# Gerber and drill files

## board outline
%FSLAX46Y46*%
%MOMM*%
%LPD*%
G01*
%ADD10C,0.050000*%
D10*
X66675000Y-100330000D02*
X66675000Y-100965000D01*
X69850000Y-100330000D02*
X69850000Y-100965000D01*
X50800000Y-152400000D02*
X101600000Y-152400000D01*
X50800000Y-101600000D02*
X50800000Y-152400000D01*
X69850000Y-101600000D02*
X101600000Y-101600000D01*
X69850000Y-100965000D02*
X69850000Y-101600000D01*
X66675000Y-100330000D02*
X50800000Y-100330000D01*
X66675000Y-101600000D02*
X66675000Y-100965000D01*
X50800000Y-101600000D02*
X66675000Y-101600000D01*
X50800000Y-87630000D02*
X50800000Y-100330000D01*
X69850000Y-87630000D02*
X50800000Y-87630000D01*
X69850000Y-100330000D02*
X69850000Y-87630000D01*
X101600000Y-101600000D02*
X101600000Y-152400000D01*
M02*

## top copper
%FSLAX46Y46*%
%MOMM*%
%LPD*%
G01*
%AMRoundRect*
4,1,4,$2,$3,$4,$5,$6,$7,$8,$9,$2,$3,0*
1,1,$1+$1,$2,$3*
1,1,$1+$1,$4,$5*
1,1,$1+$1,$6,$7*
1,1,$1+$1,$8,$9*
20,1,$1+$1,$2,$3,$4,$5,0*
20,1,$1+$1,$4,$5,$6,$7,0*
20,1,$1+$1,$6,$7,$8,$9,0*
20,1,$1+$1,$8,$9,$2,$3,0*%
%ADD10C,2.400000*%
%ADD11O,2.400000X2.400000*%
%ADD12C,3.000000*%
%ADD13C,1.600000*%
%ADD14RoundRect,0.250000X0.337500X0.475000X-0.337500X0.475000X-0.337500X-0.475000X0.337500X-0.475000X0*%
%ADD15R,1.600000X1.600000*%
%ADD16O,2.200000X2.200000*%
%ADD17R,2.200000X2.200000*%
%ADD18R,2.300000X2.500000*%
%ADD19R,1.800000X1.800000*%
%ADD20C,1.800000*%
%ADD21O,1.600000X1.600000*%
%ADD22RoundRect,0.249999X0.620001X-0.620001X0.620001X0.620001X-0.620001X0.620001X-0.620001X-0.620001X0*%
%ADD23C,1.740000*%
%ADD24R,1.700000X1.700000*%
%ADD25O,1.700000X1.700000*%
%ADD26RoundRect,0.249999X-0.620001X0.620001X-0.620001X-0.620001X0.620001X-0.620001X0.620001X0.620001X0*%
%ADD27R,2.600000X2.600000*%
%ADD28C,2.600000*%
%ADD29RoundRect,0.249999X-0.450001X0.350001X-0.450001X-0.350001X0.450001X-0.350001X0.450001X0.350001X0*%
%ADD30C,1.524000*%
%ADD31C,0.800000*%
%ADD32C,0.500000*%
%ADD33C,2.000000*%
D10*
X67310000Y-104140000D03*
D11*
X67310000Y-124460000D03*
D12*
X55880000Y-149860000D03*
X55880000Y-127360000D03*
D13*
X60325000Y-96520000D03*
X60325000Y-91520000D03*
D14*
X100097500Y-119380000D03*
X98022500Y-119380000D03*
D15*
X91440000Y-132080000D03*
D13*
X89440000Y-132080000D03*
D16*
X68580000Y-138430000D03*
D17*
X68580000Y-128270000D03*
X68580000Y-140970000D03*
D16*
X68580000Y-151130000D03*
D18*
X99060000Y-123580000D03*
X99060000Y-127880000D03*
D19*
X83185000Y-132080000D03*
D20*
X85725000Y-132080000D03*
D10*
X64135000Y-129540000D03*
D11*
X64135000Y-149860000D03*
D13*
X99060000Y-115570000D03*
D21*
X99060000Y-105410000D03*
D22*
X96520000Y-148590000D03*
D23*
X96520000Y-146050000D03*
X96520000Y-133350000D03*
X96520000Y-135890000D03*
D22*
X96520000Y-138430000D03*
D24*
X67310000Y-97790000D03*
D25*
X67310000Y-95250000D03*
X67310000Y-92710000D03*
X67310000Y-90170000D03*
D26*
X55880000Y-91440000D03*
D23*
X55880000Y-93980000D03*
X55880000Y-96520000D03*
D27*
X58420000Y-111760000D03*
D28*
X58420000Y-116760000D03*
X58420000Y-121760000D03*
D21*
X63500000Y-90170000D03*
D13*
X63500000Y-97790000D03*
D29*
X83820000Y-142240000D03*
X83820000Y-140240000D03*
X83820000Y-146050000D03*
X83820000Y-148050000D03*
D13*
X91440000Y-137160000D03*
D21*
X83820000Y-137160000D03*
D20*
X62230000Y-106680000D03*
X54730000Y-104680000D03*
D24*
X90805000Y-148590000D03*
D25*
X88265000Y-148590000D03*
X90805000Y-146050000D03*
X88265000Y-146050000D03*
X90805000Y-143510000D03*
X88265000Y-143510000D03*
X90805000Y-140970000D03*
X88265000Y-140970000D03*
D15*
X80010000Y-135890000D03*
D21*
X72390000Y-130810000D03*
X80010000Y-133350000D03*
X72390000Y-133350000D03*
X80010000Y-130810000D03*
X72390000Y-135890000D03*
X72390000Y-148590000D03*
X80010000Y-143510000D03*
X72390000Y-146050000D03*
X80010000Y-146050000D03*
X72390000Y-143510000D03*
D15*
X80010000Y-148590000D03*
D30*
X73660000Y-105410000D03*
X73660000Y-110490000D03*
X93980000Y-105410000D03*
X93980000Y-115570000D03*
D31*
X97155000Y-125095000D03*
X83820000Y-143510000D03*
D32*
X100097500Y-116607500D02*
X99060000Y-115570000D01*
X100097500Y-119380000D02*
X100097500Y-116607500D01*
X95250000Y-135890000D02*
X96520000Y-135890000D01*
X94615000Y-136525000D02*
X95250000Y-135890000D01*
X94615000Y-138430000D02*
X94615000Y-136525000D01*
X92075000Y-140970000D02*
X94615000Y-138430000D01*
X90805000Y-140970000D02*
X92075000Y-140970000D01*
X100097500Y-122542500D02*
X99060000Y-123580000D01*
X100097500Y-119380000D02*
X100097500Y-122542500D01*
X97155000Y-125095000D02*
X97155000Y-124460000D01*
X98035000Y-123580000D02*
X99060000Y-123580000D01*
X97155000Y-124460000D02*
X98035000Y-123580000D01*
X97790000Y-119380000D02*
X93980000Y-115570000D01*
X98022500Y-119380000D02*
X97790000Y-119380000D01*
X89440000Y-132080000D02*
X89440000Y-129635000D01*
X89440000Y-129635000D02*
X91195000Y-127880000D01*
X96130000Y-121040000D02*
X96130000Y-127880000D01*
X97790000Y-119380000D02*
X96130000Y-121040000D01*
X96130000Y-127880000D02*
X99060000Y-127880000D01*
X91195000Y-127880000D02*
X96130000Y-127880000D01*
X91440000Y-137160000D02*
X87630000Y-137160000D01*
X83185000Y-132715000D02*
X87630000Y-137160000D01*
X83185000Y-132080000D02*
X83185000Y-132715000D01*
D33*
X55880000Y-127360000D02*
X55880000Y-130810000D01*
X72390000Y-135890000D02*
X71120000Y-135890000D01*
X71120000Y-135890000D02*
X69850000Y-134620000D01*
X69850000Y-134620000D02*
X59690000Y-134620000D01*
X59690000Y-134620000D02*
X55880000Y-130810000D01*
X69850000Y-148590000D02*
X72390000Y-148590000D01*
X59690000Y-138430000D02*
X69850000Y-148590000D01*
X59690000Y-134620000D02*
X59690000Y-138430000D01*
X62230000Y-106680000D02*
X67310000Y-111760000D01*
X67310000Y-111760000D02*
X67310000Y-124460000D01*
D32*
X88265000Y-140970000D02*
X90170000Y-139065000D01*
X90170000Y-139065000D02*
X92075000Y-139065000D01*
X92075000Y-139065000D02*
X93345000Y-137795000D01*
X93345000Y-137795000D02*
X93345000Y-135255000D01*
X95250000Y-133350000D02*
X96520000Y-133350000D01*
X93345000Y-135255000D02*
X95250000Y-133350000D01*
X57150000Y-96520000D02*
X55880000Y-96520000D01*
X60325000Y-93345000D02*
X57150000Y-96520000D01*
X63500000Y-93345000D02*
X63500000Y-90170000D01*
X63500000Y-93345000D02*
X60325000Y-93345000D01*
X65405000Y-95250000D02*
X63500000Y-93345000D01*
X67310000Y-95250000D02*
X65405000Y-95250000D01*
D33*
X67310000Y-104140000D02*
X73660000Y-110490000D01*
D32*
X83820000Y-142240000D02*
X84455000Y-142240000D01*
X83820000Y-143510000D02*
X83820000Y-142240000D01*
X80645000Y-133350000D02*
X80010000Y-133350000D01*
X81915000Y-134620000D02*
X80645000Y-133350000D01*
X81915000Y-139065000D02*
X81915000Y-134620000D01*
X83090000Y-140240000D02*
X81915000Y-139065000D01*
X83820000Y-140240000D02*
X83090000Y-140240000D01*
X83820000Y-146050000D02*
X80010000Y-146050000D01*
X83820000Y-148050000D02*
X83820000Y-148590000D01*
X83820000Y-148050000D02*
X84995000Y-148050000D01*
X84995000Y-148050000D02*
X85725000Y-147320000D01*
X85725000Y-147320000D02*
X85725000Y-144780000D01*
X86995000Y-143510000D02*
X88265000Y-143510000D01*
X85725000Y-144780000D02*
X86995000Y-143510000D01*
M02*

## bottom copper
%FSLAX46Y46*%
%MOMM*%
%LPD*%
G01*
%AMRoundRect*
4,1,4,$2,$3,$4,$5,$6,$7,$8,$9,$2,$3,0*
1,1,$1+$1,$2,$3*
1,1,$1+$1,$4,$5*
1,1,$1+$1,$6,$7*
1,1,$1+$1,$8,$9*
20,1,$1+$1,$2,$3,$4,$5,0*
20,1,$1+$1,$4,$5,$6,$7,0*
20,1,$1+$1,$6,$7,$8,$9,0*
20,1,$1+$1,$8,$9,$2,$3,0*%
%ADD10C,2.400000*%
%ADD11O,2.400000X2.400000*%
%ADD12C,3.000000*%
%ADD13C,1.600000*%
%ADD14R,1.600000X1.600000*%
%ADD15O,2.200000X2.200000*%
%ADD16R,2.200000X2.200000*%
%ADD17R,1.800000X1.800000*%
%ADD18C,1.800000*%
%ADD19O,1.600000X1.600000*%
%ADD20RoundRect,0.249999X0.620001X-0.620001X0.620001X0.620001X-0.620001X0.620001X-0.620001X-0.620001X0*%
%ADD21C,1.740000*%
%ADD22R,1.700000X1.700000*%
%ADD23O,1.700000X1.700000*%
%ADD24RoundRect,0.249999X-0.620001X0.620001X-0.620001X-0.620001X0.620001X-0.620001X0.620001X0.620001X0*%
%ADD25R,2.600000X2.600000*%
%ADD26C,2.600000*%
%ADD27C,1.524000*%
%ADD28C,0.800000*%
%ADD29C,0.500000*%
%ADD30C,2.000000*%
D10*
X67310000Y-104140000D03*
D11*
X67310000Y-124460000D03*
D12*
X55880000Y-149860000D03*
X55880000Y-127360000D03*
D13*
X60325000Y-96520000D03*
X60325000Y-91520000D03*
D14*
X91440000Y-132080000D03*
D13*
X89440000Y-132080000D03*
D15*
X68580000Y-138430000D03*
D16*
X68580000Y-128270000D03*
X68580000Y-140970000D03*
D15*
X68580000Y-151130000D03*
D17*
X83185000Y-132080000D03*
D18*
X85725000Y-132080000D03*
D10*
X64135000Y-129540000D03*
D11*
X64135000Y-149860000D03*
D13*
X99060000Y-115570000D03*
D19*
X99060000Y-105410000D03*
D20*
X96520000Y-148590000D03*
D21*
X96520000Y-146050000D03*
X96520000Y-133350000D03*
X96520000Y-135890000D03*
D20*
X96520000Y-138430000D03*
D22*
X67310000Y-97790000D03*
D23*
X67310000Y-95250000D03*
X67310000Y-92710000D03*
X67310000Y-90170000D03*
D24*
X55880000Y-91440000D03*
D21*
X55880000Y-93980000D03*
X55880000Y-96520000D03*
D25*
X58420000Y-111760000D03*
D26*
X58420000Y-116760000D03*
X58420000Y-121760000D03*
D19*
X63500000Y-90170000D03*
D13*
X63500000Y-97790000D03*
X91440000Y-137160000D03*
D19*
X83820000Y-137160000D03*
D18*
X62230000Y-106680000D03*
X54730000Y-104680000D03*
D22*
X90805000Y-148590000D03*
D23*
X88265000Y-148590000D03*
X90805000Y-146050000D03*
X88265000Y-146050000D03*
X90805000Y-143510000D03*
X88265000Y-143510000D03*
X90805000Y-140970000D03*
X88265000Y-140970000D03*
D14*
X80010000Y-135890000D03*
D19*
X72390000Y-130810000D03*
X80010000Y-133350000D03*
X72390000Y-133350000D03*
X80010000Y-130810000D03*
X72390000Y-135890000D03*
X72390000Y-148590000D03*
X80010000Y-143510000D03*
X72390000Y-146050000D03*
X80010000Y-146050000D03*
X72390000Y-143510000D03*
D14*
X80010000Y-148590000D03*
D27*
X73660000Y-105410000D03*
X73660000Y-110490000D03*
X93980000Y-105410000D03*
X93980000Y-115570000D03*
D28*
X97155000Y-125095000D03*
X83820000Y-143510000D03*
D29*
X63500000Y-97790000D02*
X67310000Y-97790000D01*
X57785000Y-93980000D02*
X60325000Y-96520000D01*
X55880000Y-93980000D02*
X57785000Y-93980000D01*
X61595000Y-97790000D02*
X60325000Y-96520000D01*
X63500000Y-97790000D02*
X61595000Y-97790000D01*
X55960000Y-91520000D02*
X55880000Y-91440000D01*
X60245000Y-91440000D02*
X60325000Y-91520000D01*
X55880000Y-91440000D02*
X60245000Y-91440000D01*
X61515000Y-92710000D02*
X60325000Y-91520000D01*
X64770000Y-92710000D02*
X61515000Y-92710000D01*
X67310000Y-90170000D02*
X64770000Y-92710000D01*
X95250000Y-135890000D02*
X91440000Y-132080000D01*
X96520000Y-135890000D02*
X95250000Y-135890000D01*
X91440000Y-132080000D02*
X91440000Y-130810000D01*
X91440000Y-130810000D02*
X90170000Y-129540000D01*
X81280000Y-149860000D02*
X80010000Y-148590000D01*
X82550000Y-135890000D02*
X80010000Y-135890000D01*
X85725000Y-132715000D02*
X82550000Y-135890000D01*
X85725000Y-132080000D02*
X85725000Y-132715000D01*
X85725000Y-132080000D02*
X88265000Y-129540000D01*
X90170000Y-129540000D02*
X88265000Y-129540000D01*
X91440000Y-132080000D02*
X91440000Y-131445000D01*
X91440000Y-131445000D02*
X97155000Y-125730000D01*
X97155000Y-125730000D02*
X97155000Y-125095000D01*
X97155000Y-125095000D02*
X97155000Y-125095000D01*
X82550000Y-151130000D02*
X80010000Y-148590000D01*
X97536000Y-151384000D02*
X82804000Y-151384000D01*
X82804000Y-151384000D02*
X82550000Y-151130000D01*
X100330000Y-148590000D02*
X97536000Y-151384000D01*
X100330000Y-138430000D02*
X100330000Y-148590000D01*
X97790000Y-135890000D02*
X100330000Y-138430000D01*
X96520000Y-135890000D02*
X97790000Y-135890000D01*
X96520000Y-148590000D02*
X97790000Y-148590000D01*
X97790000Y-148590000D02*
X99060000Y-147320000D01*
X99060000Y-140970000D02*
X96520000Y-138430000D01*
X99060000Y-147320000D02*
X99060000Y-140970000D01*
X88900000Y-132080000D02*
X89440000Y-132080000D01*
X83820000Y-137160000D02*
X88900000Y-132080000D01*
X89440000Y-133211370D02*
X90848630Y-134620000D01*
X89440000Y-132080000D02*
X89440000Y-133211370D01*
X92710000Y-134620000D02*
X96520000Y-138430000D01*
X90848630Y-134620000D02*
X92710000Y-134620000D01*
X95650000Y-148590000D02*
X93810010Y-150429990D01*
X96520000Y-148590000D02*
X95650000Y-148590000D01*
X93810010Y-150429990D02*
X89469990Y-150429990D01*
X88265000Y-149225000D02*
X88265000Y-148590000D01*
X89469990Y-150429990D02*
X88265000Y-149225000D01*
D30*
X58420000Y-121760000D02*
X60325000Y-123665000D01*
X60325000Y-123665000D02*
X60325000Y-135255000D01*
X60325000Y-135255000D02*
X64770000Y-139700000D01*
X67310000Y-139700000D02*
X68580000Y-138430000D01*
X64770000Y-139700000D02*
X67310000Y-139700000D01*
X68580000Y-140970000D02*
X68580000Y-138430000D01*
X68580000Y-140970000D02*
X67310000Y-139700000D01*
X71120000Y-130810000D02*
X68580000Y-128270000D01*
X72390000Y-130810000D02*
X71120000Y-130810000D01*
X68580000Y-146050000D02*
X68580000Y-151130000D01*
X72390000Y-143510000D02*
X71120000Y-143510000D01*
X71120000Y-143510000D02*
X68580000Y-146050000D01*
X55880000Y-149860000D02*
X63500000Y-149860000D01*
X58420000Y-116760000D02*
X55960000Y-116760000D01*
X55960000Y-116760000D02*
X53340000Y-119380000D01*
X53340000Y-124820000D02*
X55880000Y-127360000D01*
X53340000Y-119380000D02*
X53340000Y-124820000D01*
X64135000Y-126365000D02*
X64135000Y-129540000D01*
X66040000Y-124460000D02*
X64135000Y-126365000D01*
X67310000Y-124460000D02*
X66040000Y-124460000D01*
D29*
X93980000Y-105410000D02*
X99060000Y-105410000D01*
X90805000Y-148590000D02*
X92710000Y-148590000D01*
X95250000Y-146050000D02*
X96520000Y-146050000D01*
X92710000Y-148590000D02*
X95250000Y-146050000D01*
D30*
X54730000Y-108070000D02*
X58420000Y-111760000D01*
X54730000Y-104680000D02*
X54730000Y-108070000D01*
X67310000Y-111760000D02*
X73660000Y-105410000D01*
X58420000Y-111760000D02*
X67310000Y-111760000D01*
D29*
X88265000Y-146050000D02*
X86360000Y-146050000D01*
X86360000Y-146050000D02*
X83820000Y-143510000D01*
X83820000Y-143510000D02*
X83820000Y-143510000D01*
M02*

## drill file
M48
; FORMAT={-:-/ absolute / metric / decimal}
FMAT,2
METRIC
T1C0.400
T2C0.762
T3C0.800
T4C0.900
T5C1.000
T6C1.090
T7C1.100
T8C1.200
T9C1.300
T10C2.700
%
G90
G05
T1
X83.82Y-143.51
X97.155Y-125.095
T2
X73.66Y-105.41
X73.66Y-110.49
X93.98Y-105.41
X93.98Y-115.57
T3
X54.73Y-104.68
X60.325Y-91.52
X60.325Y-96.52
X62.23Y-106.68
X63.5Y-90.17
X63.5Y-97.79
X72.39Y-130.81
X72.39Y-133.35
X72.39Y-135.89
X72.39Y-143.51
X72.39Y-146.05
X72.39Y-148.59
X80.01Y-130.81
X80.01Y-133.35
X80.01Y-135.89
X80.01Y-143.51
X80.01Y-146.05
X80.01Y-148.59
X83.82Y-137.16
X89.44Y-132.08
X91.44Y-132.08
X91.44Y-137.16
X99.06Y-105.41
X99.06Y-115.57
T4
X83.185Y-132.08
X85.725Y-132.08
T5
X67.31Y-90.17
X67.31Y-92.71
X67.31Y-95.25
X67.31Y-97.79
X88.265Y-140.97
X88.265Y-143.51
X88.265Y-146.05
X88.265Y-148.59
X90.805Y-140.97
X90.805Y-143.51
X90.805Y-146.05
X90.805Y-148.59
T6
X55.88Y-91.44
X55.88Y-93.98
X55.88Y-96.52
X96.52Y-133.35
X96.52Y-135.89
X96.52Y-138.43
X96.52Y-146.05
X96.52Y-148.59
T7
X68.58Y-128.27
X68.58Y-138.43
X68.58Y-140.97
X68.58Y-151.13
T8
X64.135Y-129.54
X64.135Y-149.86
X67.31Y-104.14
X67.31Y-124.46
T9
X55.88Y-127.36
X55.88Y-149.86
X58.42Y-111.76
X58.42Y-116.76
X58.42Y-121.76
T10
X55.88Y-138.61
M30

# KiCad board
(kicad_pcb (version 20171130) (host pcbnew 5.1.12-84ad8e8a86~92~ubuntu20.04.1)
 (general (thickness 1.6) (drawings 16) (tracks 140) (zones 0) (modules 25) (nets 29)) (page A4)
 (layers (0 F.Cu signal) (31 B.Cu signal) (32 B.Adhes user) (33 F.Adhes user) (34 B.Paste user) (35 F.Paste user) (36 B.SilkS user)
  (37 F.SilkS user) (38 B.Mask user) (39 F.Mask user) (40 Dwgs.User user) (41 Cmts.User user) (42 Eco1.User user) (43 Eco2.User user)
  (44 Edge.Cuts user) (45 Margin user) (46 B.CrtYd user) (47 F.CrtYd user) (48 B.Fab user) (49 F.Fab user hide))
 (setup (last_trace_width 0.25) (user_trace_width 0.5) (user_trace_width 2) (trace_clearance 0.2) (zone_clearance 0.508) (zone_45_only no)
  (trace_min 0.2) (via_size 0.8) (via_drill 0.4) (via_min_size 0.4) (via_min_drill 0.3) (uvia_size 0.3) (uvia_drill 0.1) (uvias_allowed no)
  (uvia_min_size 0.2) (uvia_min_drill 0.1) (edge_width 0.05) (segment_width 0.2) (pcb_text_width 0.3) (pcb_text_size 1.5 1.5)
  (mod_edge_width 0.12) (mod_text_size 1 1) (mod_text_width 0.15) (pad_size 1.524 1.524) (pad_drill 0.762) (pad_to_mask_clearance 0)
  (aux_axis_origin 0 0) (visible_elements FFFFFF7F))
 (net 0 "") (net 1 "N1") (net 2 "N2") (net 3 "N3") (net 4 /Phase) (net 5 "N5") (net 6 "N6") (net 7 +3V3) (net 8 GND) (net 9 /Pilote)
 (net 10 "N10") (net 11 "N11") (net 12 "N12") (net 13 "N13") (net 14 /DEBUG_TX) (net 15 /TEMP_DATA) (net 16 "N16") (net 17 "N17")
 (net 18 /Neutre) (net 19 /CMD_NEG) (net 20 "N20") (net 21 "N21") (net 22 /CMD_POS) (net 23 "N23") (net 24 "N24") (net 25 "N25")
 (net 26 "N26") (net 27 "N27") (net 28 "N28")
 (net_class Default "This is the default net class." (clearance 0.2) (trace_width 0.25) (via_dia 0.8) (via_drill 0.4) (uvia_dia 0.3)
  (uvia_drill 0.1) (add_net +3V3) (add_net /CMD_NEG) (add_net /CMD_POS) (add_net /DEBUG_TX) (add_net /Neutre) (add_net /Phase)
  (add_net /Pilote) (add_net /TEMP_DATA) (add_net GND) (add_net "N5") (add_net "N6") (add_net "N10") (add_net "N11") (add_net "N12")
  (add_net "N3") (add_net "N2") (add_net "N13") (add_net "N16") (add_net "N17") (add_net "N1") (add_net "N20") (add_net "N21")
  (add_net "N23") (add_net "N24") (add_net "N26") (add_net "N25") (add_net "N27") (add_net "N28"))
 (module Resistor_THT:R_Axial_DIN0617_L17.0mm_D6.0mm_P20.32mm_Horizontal (layer F.Cu) (at 67.31 104.14 270)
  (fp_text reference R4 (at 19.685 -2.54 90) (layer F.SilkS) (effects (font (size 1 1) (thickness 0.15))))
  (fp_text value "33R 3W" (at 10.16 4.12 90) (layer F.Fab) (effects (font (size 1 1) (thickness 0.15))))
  (pad 1 thru_hole circle (at 0 0 270) (size 2.4 2.4) (drill 1.2) (layers *.Cu *.Mask) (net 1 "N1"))
  (pad 2 thru_hole oval (at 20.32 0 270) (size 2.4 2.4) (drill 1.2) (layers *.Cu *.Mask) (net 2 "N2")))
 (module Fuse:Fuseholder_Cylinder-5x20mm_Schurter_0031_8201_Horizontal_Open (layer F.Cu) (at 55.88 149.86 90)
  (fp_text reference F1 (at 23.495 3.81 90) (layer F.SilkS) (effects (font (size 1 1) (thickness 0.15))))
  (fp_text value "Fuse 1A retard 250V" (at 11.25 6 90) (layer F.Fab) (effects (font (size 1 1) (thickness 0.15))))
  (pad 1 thru_hole circle (at 0 0 90) (size 3 3) (drill 1.3) (layers *.Cu *.Mask) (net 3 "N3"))
  (pad 2 thru_hole circle (at 22.5 0 90) (size 3 3) (drill 1.3) (layers *.Cu *.Mask) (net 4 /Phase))
  (pad "" np_thru_hole circle (at 11.25 0 90) (size 2.7 2.7) (drill 2.7) (layers *.Cu *.Mask)))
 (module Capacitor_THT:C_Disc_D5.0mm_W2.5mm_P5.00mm (layer F.Cu) (at 60.325 96.52 90)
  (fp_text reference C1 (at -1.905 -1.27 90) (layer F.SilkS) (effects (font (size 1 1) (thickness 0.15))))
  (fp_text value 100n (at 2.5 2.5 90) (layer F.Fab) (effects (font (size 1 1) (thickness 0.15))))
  (pad 1 thru_hole circle (at 0 0 90) (size 1.6 1.6) (drill 0.8) (layers *.Cu *.Mask) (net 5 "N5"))
  (pad 2 thru_hole circle (at 5 0 90) (size 1.6 1.6) (drill 0.8) (layers *.Cu *.Mask) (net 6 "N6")))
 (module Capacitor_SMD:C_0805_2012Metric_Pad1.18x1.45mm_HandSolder (layer F.Cu) (at 99.06 119.38 180)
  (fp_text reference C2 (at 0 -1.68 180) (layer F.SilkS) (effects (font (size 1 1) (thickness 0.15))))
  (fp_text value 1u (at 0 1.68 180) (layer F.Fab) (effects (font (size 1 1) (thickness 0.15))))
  (pad 1 smd roundrect (at -1.0375 0 180) (size 1.175 1.45) (layers F.Cu F.Paste F.Mask) (roundrect_rratio 0.2127659574468085) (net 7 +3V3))
  (pad 2 smd roundrect (at 1.0375 0 180) (size 1.175 1.45) (layers F.Cu F.Paste F.Mask) (roundrect_rratio 0.2127659574468085) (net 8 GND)))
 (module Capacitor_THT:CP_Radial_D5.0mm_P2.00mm (layer F.Cu) (at 91.44 132.08 180)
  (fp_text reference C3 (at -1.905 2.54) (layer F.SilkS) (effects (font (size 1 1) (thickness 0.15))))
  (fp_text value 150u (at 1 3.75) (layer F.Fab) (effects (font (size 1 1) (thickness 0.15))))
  (pad 1 thru_hole rect (at 0 0 180) (size 1.6 1.6) (drill 0.8) (layers *.Cu *.Mask) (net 7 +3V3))
  (pad 2 thru_hole circle (at 2 0 180) (size 1.6 1.6) (drill 0.8) (layers *.Cu *.Mask) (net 8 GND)))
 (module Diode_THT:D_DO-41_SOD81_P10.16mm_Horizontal (layer F.Cu) (at 68.58 128.27 270)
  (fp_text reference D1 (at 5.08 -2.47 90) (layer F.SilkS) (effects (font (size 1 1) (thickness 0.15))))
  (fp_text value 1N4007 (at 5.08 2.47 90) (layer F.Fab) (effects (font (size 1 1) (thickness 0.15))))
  (pad 2 thru_hole oval (at 10.16 0 270) (size 2.2 2.2) (drill 1.1) (layers *.Cu *.Mask) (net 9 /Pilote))
  (pad 1 thru_hole rect (at 0 0 270) (size 2.2 2.2) (drill 1.1) (layers *.Cu *.Mask) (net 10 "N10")))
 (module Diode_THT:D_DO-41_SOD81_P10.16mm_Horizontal (layer F.Cu) (at 68.58 140.97 270)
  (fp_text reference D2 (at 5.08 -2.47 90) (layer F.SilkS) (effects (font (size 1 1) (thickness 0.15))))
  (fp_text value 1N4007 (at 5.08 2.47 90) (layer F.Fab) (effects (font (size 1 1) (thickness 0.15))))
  (pad 1 thru_hole rect (at 0 0 270) (size 2.2 2.2) (drill 1.1) (layers *.Cu *.Mask) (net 9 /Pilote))
  (pad 2 thru_hole oval (at 10.16 0 270) (size 2.2 2.2) (drill 1.1) (layers *.Cu *.Mask) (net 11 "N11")))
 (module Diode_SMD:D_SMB (layer F.Cu) (at 99.06 125.73 270)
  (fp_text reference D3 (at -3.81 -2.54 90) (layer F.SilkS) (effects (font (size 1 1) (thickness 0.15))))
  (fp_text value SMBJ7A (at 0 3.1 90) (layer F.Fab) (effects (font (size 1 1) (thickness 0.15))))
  (pad 1 smd rect (at -2.15 0 270) (size 2.5 2.3) (layers F.Cu F.Paste F.Mask) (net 7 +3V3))
  (pad 2 smd rect (at 2.15 0 270) (size 2.5 2.3) (layers F.Cu F.Paste F.Mask) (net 8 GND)))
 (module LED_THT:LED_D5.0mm (layer F.Cu) (at 83.185 132.08)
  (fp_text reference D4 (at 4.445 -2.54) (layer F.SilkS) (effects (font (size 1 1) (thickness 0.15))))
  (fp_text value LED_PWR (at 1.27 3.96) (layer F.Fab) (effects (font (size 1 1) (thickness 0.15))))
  (pad 1 thru_hole rect (at 0 0) (size 1.8 1.8) (drill 0.9) (layers *.Cu *.Mask) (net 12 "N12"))
  (pad 2 thru_hole circle (at 2.54 0) (size 1.8 1.8) (drill 0.9) (layers *.Cu *.Mask) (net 7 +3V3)))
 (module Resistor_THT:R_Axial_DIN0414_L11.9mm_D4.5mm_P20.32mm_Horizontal (layer F.Cu) (at 64.135 129.54 270)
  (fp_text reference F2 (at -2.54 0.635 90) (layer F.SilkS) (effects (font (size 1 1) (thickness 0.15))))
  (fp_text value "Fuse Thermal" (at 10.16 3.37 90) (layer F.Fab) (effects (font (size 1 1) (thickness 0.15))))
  (pad 1 thru_hole circle (at 0 0 270) (size 2.4 2.4) (drill 1.2) (layers *.Cu *.Mask) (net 2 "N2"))
  (pad 2 thru_hole oval (at 20.32 0 270) (size 2.4 2.4) (drill 1.2) (layers *.Cu *.Mask) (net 3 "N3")))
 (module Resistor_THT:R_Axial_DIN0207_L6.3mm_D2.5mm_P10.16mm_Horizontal (layer F.Cu) (at 99.06 115.57 90)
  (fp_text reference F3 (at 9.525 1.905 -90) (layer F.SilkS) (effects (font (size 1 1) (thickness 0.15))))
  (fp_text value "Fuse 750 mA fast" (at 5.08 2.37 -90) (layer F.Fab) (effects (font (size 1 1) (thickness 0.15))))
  (pad 1 thru_hole circle (at 0 0 90) (size 1.6 1.6) (drill 0.8) (layers *.Cu *.Mask) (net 7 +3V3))
  (pad 2 thru_hole oval (at 10.16 0 90) (size 1.6 1.6) (drill 0.8) (layers *.Cu *.Mask) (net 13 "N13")))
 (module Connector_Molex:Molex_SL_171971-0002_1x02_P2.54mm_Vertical (layer F.Cu) (at 96.52 148.59 90)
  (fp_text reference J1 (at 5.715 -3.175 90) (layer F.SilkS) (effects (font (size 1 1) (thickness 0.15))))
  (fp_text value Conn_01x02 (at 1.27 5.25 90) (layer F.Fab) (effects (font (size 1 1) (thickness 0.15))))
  (pad 1 thru_hole roundrect (at 0 0 90) (size 1.74 1.74) (drill 1.09) (layers *.Cu *.Mask) (roundrect_rratio 0.1436775862068966)
   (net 8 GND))
  (pad 2 thru_hole circle (at 2.54 0 90) (size 1.74 1.74) (drill 1.09) (layers *.Cu *.Mask) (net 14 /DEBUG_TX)))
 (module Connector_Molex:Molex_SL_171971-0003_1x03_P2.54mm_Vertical (layer F.Cu) (at 96.52 138.43 90)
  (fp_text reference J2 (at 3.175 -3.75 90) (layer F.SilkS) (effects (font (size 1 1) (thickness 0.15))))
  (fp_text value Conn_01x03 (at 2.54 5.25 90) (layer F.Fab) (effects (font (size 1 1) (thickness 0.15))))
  (pad 3 thru_hole circle (at 5.08 0 90) (size 1.74 1.74) (drill 1.09) (layers *.Cu *.Mask) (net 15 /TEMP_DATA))
  (pad 2 thru_hole circle (at 2.54 0 90) (size 1.74 1.74) (drill 1.09) (layers *.Cu *.Mask) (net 7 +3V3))
  (pad 1 thru_hole roundrect (at 0 0 90) (size 1.74 1.74) (drill 1.09) (layers *.Cu *.Mask) (roundrect_rratio 0.1436775862068966)
   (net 8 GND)))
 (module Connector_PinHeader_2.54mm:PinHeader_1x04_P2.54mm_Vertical (layer F.Cu) (at 67.31 97.79 180)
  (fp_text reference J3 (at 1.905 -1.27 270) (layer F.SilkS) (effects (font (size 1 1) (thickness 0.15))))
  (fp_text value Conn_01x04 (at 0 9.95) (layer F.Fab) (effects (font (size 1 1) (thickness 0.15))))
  (pad 1 thru_hole rect (at 0 0 180) (size 1.7 1.7) (drill 1) (layers *.Cu *.Mask) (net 5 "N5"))
  (pad 2 thru_hole oval (at 0 2.54 180) (size 1.7 1.7) (drill 1) (layers *.Cu *.Mask) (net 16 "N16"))
  (pad 3 thru_hole oval (at 0 5.08 180) (size 1.7 1.7) (drill 1) (layers *.Cu *.Mask) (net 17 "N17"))
  (pad 4 thru_hole oval (at 0 7.62 180) (size 1.7 1.7) (drill 1) (layers *.Cu *.Mask) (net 6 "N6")))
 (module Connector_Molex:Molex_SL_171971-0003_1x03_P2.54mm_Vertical (layer F.Cu) (at 55.88 91.44 270)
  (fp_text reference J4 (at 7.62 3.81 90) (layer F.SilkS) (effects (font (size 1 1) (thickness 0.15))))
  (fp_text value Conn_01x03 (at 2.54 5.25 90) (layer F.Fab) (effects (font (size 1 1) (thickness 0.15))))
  (pad 1 thru_hole roundrect (at 0 0 270) (size 1.74 1.74) (drill 1.09) (layers *.Cu *.Mask) (roundrect_rratio 0.1436775862068966)
   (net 6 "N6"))
  (pad 2 thru_hole circle (at 2.54 0 270) (size 1.74 1.74) (drill 1.09) (layers *.Cu *.Mask) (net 5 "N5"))
  (pad 3 thru_hole circle (at 5.08 0 270) (size 1.74 1.74) (drill 1.09) (layers *.Cu *.Mask) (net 16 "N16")))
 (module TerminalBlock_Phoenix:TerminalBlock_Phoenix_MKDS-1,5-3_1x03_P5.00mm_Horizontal (layer F.Cu) (at 58.42 111.76 270)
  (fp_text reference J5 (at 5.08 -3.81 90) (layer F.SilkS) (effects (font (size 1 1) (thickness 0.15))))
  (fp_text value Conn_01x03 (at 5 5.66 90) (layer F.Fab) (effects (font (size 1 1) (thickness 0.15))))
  (pad 1 thru_hole rect (at 0 0 270) (size 2.6 2.6) (drill 1.3) (layers *.Cu *.Mask) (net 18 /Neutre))
  (pad 2 thru_hole circle (at 5 0 270) (size 2.6 2.6) (drill 1.3) (layers *.Cu *.Mask) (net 4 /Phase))
  (pad 3 thru_hole circle (at 10 0 270) (size 2.6 2.6) (drill 1.3) (layers *.Cu *.Mask) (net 9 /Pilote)))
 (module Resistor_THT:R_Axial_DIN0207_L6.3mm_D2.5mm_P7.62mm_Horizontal (layer F.Cu) (at 63.5 97.79 90)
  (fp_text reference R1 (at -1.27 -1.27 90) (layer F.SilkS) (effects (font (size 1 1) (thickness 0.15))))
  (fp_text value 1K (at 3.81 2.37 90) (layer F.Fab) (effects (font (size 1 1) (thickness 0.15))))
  (pad 2 thru_hole oval (at 7.62 0 90) (size 1.6 1.6) (drill 0.8) (layers *.Cu *.Mask) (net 16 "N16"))
  (pad 1 thru_hole circle (at 0 0 90) (size 1.6 1.6) (drill 0.8) (layers *.Cu *.Mask) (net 5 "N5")))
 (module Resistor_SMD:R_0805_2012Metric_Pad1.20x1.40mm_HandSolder (layer F.Cu) (at 83.82 141.24 270)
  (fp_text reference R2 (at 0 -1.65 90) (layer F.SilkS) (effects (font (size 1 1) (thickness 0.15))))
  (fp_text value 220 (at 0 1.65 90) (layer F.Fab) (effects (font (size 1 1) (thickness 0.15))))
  (pad 2 smd roundrect (at 1 0 270) (size 1.2 1.4) (layers F.Cu F.Paste F.Mask) (roundrect_rratio 0.2083325) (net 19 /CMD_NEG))
  (pad 1 smd roundrect (at -1 0 270) (size 1.2 1.4) (layers F.Cu F.Paste F.Mask) (roundrect_rratio 0.2083325) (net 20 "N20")))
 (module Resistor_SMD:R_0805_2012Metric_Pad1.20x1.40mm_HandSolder (layer F.Cu) (at 83.82 147.05 270)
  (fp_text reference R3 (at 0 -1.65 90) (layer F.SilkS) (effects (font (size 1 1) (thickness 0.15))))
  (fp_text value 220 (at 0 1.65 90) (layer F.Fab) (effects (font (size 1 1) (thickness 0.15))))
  (pad 1 smd roundrect (at -1 0 270) (size 1.2 1.4) (layers F.Cu F.Paste F.Mask) (roundrect_rratio 0.2083325) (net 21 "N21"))
  (pad 2 smd roundrect (at 1 0 270) (size 1.2 1.4) (layers F.Cu F.Paste F.Mask) (roundrect_rratio 0.2083325) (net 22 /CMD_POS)))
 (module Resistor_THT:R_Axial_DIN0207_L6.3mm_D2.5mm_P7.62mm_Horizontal (layer F.Cu) (at 91.44 137.16 180)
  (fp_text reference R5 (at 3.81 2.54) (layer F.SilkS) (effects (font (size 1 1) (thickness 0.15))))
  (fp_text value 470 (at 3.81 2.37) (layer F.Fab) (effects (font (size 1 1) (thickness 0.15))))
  (pad 1 thru_hole circle (at 0 0 180) (size 1.6 1.6) (drill 0.8) (layers *.Cu *.Mask) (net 12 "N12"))
  (pad 2 thru_hole oval (at 7.62 0 180) (size 1.6 1.6) (drill 0.8) (layers *.Cu *.Mask) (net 8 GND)))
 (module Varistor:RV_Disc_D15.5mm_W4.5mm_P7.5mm (layer F.Cu) (at 62.23 106.68 180)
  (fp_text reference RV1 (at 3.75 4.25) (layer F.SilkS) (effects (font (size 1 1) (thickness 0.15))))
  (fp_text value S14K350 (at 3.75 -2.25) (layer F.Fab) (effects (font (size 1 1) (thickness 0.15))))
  (pad 1 thru_hole circle (at 0 0 180) (size 1.8 1.8) (drill 0.8) (layers *.Cu *.Mask) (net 2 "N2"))
  (pad 2 thru_hole circle (at 7.5 2 180) (size 1.8 1.8) (drill 0.8) (layers *.Cu *.Mask) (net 18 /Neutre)))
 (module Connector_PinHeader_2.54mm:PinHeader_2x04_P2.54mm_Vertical (layer F.Cu) (at 90.805 148.59 180)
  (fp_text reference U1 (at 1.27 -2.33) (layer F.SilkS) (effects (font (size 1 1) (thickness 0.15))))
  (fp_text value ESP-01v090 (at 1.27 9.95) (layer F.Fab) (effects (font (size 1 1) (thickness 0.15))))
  (pad 1 thru_hole rect (at 0 0 180) (size 1.7 1.7) (drill 1) (layers *.Cu *.Mask) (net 14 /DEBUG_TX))
  (pad 2 thru_hole oval (at 2.54 0 180) (size 1.7 1.7) (drill 1) (layers *.Cu *.Mask) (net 8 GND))
  (pad 3 thru_hole oval (at 0 2.54 180) (size 1.7 1.7) (drill 1) (layers *.Cu *.Mask) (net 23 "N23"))
  (pad 4 thru_hole oval (at 2.54 2.54 180) (size 1.7 1.7) (drill 1) (layers *.Cu *.Mask) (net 19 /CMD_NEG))
  (pad 5 thru_hole oval (at 0 5.08 180) (size 1.7 1.7) (drill 1) (layers *.Cu *.Mask) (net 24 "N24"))
  (pad 6 thru_hole oval (at 2.54 5.08 180) (size 1.7 1.7) (drill 1) (layers *.Cu *.Mask) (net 22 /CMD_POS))
  (pad 7 thru_hole oval (at 0 7.62 180) (size 1.7 1.7) (drill 1) (layers *.Cu *.Mask) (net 7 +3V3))
  (pad 8 thru_hole oval (at 2.54 7.62 180) (size 1.7 1.7) (drill 1) (layers *.Cu *.Mask) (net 15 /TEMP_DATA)))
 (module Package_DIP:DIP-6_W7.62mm (layer F.Cu) (at 80.01 135.89 180)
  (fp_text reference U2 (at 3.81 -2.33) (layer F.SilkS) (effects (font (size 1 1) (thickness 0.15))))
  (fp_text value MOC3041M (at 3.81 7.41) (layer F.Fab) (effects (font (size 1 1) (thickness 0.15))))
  (pad 1 thru_hole rect (at 0 0 180) (size 1.6 1.6) (drill 0.8) (layers *.Cu *.Mask) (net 7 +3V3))
  (pad 4 thru_hole oval (at 7.62 5.08 180) (size 1.6 1.6) (drill 0.8) (layers *.Cu *.Mask) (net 10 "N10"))
  (pad 2 thru_hole oval (at 0 2.54 180) (size 1.6 1.6) (drill 0.8) (layers *.Cu *.Mask) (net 20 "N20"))
  (pad 5 thru_hole oval (at 7.62 2.54 180) (size 1.6 1.6) (drill 0.8) (layers *.Cu *.Mask) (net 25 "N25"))
  (pad 3 thru_hole oval (at 0 5.08 180) (size 1.6 1.6) (drill 0.8) (layers *.Cu *.Mask) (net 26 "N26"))
  (pad 6 thru_hole oval (at 7.62 0 180) (size 1.6 1.6) (drill 0.8) (layers *.Cu *.Mask) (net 4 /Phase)))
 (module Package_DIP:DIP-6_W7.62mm (layer F.Cu) (at 80.01 148.59 180)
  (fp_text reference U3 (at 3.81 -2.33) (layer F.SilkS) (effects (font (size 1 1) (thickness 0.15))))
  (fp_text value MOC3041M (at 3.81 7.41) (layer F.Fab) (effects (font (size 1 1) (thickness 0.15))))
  (pad 6 thru_hole oval (at 7.62 0 180) (size 1.6 1.6) (drill 0.8) (layers *.Cu *.Mask) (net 4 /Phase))
  (pad 3 thru_hole oval (at 0 5.08 180) (size 1.6 1.6) (drill 0.8) (layers *.Cu *.Mask) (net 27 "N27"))
  (pad 5 thru_hole oval (at 7.62 2.54 180) (size 1.6 1.6) (drill 0.8) (layers *.Cu *.Mask) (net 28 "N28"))
  (pad 2 thru_hole oval (at 0 2.54 180) (size 1.6 1.6) (drill 0.8) (layers *.Cu *.Mask) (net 21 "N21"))
  (pad 4 thru_hole oval (at 7.62 5.08 180) (size 1.6 1.6) (drill 0.8) (layers *.Cu *.Mask) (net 11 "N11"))
  (pad 1 thru_hole rect (at 0 0 180) (size 1.6 1.6) (drill 0.8) (layers *.Cu *.Mask) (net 7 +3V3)))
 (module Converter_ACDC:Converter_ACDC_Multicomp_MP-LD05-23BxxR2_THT (layer F.Cu) (at 83.82 115.57)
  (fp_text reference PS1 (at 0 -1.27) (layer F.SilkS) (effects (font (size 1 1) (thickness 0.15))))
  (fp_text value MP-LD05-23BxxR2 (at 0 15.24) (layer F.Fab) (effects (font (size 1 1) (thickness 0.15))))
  (pad 1 thru_hole circle (at -10.16 -10.16) (size 1.524 1.524) (drill 0.762) (layers *.Cu *.Mask) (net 18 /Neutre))
  (pad 2 thru_hole circle (at -10.16 -5.08) (size 1.524 1.524) (drill 0.762) (layers *.Cu *.Mask) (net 1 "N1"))
  (pad 5 thru_hole circle (at 10.16 -10.16) (size 1.524 1.524) (drill 0.762) (layers *.Cu *.Mask) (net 13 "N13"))
  (pad 4 thru_hole circle (at 10.16 0) (size 1.524 1.524) (drill 0.762) (layers *.Cu *.Mask) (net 8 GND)))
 (gr_line (start 66.675 100.33) (end 66.675 100.965) (layer Edge.Cuts) (width 0.05))
 (gr_line (start 69.85 100.33) (end 69.85 100.965) (layer Edge.Cuts) (width 0.05))
 (gr_line (start 50.8 152.4) (end 101.6 152.4) (layer Edge.Cuts) (width 0.05))
 (gr_line (start 50.8 101.6) (end 50.8 152.4) (layer Edge.Cuts) (width 0.05))
 (gr_line (start 69.85 101.6) (end 101.6 101.6) (layer Edge.Cuts) (width 0.05))
 (gr_line (start 69.85 100.965) (end 69.85 101.6) (layer Edge.Cuts) (width 0.05))
 (gr_line (start 66.675 100.33) (end 50.8 100.33) (layer Edge.Cuts) (width 0.05))
 (gr_line (start 66.675 101.6) (end 66.675 100.965) (layer Edge.Cuts) (width 0.05))
 (gr_line (start 50.8 101.6) (end 66.675 101.6) (layer Edge.Cuts) (width 0.05))
 (gr_line (start 50.8 87.63) (end 50.8 100.33) (layer Edge.Cuts) (width 0.05))
 (gr_line (start 69.85 87.63) (end 50.8 87.63) (layer Edge.Cuts) (width 0.05))
 (gr_line (start 69.85 100.33) (end 69.85 87.63) (layer Edge.Cuts) (width 0.05))
 (gr_line (start 101.6 101.6) (end 101.6 152.4) (layer Edge.Cuts) (width 0.05))
 (segment (start 63.5 97.79) (end 67.31 97.79) (width 0.5) (layer B.Cu) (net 5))
 (segment (start 57.785 93.98) (end 60.325 96.52) (width 0.5) (layer B.Cu) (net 5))
 (segment (start 55.88 93.98) (end 57.785 93.98) (width 0.5) (layer B.Cu) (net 5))
 (segment (start 61.595 97.79) (end 60.325 96.52) (width 0.5) (layer B.Cu) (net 5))
 (segment (start 63.5 97.79) (end 61.595 97.79) (width 0.5) (layer B.Cu) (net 5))
 (segment (start 55.96 91.52) (end 55.88 91.44) (width 0.5) (layer B.Cu) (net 6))
 (segment (start 60.245 91.44) (end 60.325 91.52) (width 0.5) (layer B.Cu) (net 6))
 (segment (start 55.88 91.44) (end 60.245 91.44) (width 0.5) (layer B.Cu) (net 6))
 (segment (start 61.515 92.71) (end 60.325 91.52) (width 0.5) (layer B.Cu) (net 6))
 (segment (start 64.77 92.71) (end 61.515 92.71) (width 0.5) (layer B.Cu) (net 6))
 (segment (start 67.31 90.17) (end 64.77 92.71) (width 0.5) (layer B.Cu) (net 6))
 (segment (start 100.0975 116.6075) (end 99.06 115.57) (width 0.5) (layer F.Cu) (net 7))
 (segment (start 100.0975 119.38) (end 100.0975 116.6075) (width 0.5) (layer F.Cu) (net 7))
 (segment (start 95.25 135.89) (end 91.44 132.08) (width 0.5) (layer B.Cu) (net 7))
 (segment (start 96.52 135.89) (end 95.25 135.89) (width 0.5) (layer B.Cu) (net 7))
 (segment (start 91.44 132.08) (end 91.44 130.81) (width 0.5) (layer B.Cu) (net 7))
 (segment (start 91.44 130.81) (end 90.17 129.54) (width 0.5) (layer B.Cu) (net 7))
 (segment (start 81.28 149.86) (end 80.01 148.59) (width 0.5) (layer B.Cu) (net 7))
 (segment (start 95.25 135.89) (end 96.52 135.89) (width 0.5) (layer F.Cu) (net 7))
 (segment (start 94.615 136.525) (end 95.25 135.89) (width 0.5) (layer F.Cu) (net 7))
 (segment (start 94.615 138.43) (end 94.615 136.525) (width 0.5) (layer F.Cu) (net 7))
 (segment (start 92.075 140.97) (end 94.615 138.43) (width 0.5) (layer F.Cu) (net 7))
 (segment (start 90.805 140.97) (end 92.075 140.97) (width 0.5) (layer F.Cu) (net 7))
 (segment (start 82.55 135.89) (end 80.01 135.89) (width 0.5) (layer B.Cu) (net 7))
 (segment (start 85.725 132.715) (end 82.55 135.89) (width 0.5) (layer B.Cu) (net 7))
 (segment (start 85.725 132.08) (end 85.725 132.715) (width 0.5) (layer B.Cu) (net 7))
 (segment (start 85.725 132.08) (end 88.265 129.54) (width 0.5) (layer B.Cu) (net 7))
 (segment (start 90.17 129.54) (end 88.265 129.54) (width 0.5) (layer B.Cu) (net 7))
 (segment (start 100.0975 122.5425) (end 99.06 123.58) (width 0.5) (layer F.Cu) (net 7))
 (segment (start 100.0975 119.38) (end 100.0975 122.5425) (width 0.5) (layer F.Cu) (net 7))
 (segment (start 91.44 132.08) (end 91.44 131.445) (width 0.5) (layer B.Cu) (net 7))
 (segment (start 91.44 131.445) (end 97.155 125.73) (width 0.5) (layer B.Cu) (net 7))
 (segment (start 97.155 125.73) (end 97.155 125.095) (width 0.5) (layer B.Cu) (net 7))
 (segment (start 97.155 125.095) (end 97.155 125.095) (width 0.5) (layer B.Cu) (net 7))
 (via (at 97.155 125.095) (size 0.8) (drill 0.4) (layers F.Cu B.Cu) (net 7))
 (segment (start 97.155 125.095) (end 97.155 124.46) (width 0.5) (layer F.Cu) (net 7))
 (segment (start 98.035 123.58) (end 99.06 123.58) (width 0.5) (layer F.Cu) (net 7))
 (segment (start 97.155 124.46) (end 98.035 123.58) (width 0.5) (layer F.Cu) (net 7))
 (segment (start 82.55 151.13) (end 80.01 148.59) (width 0.5) (layer B.Cu) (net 7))
 (segment (start 97.536 151.384) (end 82.804 151.384) (width 0.5) (layer B.Cu) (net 7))
 (segment (start 82.804 151.384) (end 82.55 151.13) (width 0.5) (layer B.Cu) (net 7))
 (segment (start 100.33 148.59) (end 97.536 151.384) (width 0.5) (layer B.Cu) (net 7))
 (segment (start 100.33 138.43) (end 100.33 148.59) (width 0.5) (layer B.Cu) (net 7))
 (segment (start 97.79 135.89) (end 100.33 138.43) (width 0.5) (layer B.Cu) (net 7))
 (segment (start 96.52 135.89) (end 97.79 135.89) (width 0.5) (layer B.Cu) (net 7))
 (segment (start 97.79 119.38) (end 93.98 115.57) (width 0.5) (layer F.Cu) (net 8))
 (segment (start 98.0225 119.38) (end 97.79 119.38) (width 0.5) (layer F.Cu) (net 8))
 (segment (start 96.52 148.59) (end 97.79 148.59) (width 0.5) (layer B.Cu) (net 8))
 (segment (start 97.79 148.59) (end 99.06 147.32) (width 0.5) (layer B.Cu) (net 8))
 (segment (start 99.06 140.97) (end 96.52 138.43) (width 0.5) (layer B.Cu) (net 8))
 (segment (start 99.06 147.32) (end 99.06 140.97) (width 0.5) (layer B.Cu) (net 8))
 (segment (start 88.9 132.08) (end 89.44 132.08) (width 0.5) (layer B.Cu) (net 8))
 (segment (start 83.82 137.16) (end 88.9 132.08) (width 0.5) (layer B.Cu) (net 8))
 (segment (start 89.44 133.21137) (end 90.84863 134.62) (width 0.5) (layer B.Cu) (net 8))
 (segment (start 89.44 132.08) (end 89.44 133.21137) (width 0.5) (layer B.Cu) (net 8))
 (segment (start 92.71 134.62) (end 96.52 138.43) (width 0.5) (layer B.Cu) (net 8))
 (segment (start 90.84863 134.62) (end 92.71 134.62) (width 0.5) (layer B.Cu) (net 8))
 (segment (start 95.65 148.59) (end 93.81001 150.42999) (width 0.5) (layer B.Cu) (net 8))
 (segment (start 96.52 148.59) (end 95.65 148.59) (width 0.5) (layer B.Cu) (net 8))
 (segment (start 93.81001 150.42999) (end 89.46999 150.42999) (width 0.5) (layer B.Cu) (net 8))
 (segment (start 88.265 149.225) (end 88.265 148.59) (width 0.5) (layer B.Cu) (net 8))
 (segment (start 89.46999 150.42999) (end 88.265 149.225) (width 0.5) (layer B.Cu) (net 8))
 (segment (start 89.44 132.08) (end 89.44 129.635) (width 0.5) (layer F.Cu) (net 8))
 (segment (start 89.44 129.635) (end 91.195 127.88) (width 0.5) (layer F.Cu) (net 8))
 (segment (start 96.13 121.04) (end 96.13 127.88) (width 0.5) (layer F.Cu) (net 8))
 (segment (start 97.79 119.38) (end 96.13 121.04) (width 0.5) (layer F.Cu) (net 8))
 (segment (start 96.13 127.88) (end 99.06 127.88) (width 0.5) (layer F.Cu) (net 8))
 (segment (start 91.195 127.88) (end 96.13 127.88) (width 0.5) (layer F.Cu) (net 8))
 (segment (start 58.42 121.76) (end 60.325 123.665) (width 2) (layer B.Cu) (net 9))
 (segment (start 60.325 123.665) (end 60.325 135.255) (width 2) (layer B.Cu) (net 9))
 (segment (start 60.325 135.255) (end 64.77 139.7) (width 2) (layer B.Cu) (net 9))
 (segment (start 67.31 139.7) (end 68.58 138.43) (width 2) (layer B.Cu) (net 9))
 (segment (start 64.77 139.7) (end 67.31 139.7) (width 2) (layer B.Cu) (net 9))
 (segment (start 68.58 140.97) (end 68.58 138.43) (width 2) (layer B.Cu) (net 9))
 (segment (start 68.58 140.97) (end 67.31 139.7) (width 2) (layer B.Cu) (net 9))
 (segment (start 71.12 130.81) (end 68.58 128.27) (width 2) (layer B.Cu) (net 10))
 (segment (start 72.39 130.81) (end 71.12 130.81) (width 2) (layer B.Cu) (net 10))
 (segment (start 68.58 146.05) (end 68.58 151.13) (width 2) (layer B.Cu) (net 11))
 (segment (start 72.39 143.51) (end 71.12 143.51) (width 2) (layer B.Cu) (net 11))
 (segment (start 71.12 143.51) (end 68.58 146.05) (width 2) (layer B.Cu) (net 11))
 (segment (start 91.44 137.16) (end 87.63 137.16) (width 0.5) (layer F.Cu) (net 12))
 (segment (start 83.185 132.715) (end 87.63 137.16) (width 0.5) (layer F.Cu) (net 12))
 (segment (start 83.185 132.08) (end 83.185 132.715) (width 0.5) (layer F.Cu) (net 12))
 (segment (start 55.88 149.86) (end 63.5 149.86) (width 2) (layer B.Cu) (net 3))
 (segment (start 58.42 116.76) (end 55.96 116.76) (width 2) (layer B.Cu) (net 4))
 (segment (start 55.96 116.76) (end 53.34 119.38) (width 2) (layer B.Cu) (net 4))
 (segment (start 53.34 124.82) (end 55.88 127.36) (width 2) (layer B.Cu) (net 4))
 (segment (start 53.34 119.38) (end 53.34 124.82) (width 2) (layer B.Cu) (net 4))
 (segment (start 55.88 127.36) (end 55.88 130.81) (width 2) (layer F.Cu) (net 4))
 (segment (start 72.39 135.89) (end 71.12 135.89) (width 2) (layer F.Cu) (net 4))
 (segment (start 71.12 135.89) (end 69.85 134.62) (width 2) (layer F.Cu) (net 4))
 (segment (start 69.85 134.62) (end 59.69 134.62) (width 2) (layer F.Cu) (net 4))
 (segment (start 59.69 134.62) (end 55.88 130.81) (width 2) (layer F.Cu) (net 4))
 (segment (start 69.85 148.59) (end 72.39 148.59) (width 2) (layer F.Cu) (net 4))
 (segment (start 59.69 138.43) (end 69.85 148.59) (width 2) (layer F.Cu) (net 4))
 (segment (start 59.69 134.62) (end 59.69 138.43) (width 2) (layer F.Cu) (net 4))
 (segment (start 62.23 106.68) (end 67.31 111.76) (width 2) (layer F.Cu) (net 2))
 (segment (start 67.31 111.76) (end 67.31 124.46) (width 2) (layer F.Cu) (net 2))
 (segment (start 64.135 126.365) (end 64.135 129.54) (width 2) (layer B.Cu) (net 2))
 (segment (start 66.04 124.46) (end 64.135 126.365) (width 2) (layer B.Cu) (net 2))
 (segment (start 67.31 124.46) (end 66.04 124.46) (width 2) (layer B.Cu) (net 2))
 (segment (start 93.98 105.41) (end 99.06 105.41) (width 0.5) (layer B.Cu) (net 13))
 (segment (start 90.805 148.59) (end 92.71 148.59) (width 0.5) (layer B.Cu) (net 14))
 (segment (start 95.25 146.05) (end 96.52 146.05) (width 0.5) (layer B.Cu) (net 14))
 (segment (start 92.71 148.59) (end 95.25 146.05) (width 0.5) (layer B.Cu) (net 14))
 (segment (start 88.265 140.97) (end 90.17 139.065) (width 0.5) (layer F.Cu) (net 15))
 (segment (start 90.17 139.065) (end 92.075 139.065) (width 0.5) (layer F.Cu) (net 15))
 (segment (start 92.075 139.065) (end 93.345 137.795) (width 0.5) (layer F.Cu) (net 15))
 (segment (start 93.345 137.795) (end 93.345 135.255) (width 0.5) (layer F.Cu) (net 15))
 (segment (start 95.25 133.35) (end 96.52 133.35) (width 0.5) (layer F.Cu) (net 15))
 (segment (start 93.345 135.255) (end 95.25 133.35) (width 0.5) (layer F.Cu) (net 15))
 (segment (start 57.15 96.52) (end 55.88 96.52) (width 0.5) (layer F.Cu) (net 16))
 (segment (start 60.325 93.345) (end 57.15 96.52) (width 0.5) (layer F.Cu) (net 16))
 (segment (start 63.5 93.345) (end 63.5 90.17) (width 0.5) (layer F.Cu) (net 16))
 (segment (start 63.5 93.345) (end 60.325 93.345) (width 0.5) (layer F.Cu) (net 16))
 (segment (start 65.405 95.25) (end 63.5 93.345) (width 0.5) (layer F.Cu) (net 16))
 (segment (start 67.31 95.25) (end 65.405 95.25) (width 0.5) (layer F.Cu) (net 16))
 (segment (start 54.73 108.07) (end 58.42 111.76) (width 2) (layer B.Cu) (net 18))
 (segment (start 54.73 104.68) (end 54.73 108.07) (width 2) (layer B.Cu) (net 18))
 (segment (start 67.31 111.76) (end 73.66 105.41) (width 2) (layer B.Cu) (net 18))
 (segment (start 58.42 111.76) (end 67.31 111.76) (width 2) (layer B.Cu) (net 18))
 (segment (start 67.31 104.14) (end 73.66 110.49) (width 2) (layer F.Cu) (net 1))
 (segment (start 83.82 142.24) (end 84.455 142.24) (width 0.5) (layer F.Cu) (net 19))
 (segment (start 88.265 146.05) (end 86.36 146.05) (width 0.5) (layer B.Cu) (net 19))
 (segment (start 86.36 146.05) (end 83.82 143.51) (width 0.5) (layer B.Cu) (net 19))
 (segment (start 83.82 143.51) (end 83.82 143.51) (width 0.5) (layer B.Cu) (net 19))
 (via (at 83.82 143.51) (size 0.8) (drill 0.4) (layers F.Cu B.Cu) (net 19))
 (segment (start 83.82 143.51) (end 83.82 142.24) (width 0.5) (layer F.Cu) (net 19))
 (segment (start 80.645 133.35) (end 80.01 133.35) (width 0.5) (layer F.Cu) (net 20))
 (segment (start 81.915 134.62) (end 80.645 133.35) (width 0.5) (layer F.Cu) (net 20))
 (segment (start 81.915 139.065) (end 81.915 134.62) (width 0.5) (layer F.Cu) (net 20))
 (segment (start 83.09 140.24) (end 81.915 139.065) (width 0.5) (layer F.Cu) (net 20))
 (segment (start 83.82 140.24) (end 83.09 140.24) (width 0.5) (layer F.Cu) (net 20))
 (segment (start 83.82 146.05) (end 80.01 146.05) (width 0.5) (layer F.Cu) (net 21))
 (segment (start 83.82 148.05) (end 83.82 148.59) (width 0.5) (layer F.Cu) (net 22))
 (segment (start 83.82 148.05) (end 84.995 148.05) (width 0.5) (layer F.Cu) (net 22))
 (segment (start 84.995 148.05) (end 85.725 147.32) (width 0.5) (layer F.Cu) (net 22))
 (segment (start 85.725 147.32) (end 85.725 144.78) (width 0.5) (layer F.Cu) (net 22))
 (segment (start 86.995 143.51) (end 88.265 143.51) (width 0.5) (layer F.Cu) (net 22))
 (segment (start 85.725 144.78) (end 86.995 143.51) (width 0.5) (layer F.Cu) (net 22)))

